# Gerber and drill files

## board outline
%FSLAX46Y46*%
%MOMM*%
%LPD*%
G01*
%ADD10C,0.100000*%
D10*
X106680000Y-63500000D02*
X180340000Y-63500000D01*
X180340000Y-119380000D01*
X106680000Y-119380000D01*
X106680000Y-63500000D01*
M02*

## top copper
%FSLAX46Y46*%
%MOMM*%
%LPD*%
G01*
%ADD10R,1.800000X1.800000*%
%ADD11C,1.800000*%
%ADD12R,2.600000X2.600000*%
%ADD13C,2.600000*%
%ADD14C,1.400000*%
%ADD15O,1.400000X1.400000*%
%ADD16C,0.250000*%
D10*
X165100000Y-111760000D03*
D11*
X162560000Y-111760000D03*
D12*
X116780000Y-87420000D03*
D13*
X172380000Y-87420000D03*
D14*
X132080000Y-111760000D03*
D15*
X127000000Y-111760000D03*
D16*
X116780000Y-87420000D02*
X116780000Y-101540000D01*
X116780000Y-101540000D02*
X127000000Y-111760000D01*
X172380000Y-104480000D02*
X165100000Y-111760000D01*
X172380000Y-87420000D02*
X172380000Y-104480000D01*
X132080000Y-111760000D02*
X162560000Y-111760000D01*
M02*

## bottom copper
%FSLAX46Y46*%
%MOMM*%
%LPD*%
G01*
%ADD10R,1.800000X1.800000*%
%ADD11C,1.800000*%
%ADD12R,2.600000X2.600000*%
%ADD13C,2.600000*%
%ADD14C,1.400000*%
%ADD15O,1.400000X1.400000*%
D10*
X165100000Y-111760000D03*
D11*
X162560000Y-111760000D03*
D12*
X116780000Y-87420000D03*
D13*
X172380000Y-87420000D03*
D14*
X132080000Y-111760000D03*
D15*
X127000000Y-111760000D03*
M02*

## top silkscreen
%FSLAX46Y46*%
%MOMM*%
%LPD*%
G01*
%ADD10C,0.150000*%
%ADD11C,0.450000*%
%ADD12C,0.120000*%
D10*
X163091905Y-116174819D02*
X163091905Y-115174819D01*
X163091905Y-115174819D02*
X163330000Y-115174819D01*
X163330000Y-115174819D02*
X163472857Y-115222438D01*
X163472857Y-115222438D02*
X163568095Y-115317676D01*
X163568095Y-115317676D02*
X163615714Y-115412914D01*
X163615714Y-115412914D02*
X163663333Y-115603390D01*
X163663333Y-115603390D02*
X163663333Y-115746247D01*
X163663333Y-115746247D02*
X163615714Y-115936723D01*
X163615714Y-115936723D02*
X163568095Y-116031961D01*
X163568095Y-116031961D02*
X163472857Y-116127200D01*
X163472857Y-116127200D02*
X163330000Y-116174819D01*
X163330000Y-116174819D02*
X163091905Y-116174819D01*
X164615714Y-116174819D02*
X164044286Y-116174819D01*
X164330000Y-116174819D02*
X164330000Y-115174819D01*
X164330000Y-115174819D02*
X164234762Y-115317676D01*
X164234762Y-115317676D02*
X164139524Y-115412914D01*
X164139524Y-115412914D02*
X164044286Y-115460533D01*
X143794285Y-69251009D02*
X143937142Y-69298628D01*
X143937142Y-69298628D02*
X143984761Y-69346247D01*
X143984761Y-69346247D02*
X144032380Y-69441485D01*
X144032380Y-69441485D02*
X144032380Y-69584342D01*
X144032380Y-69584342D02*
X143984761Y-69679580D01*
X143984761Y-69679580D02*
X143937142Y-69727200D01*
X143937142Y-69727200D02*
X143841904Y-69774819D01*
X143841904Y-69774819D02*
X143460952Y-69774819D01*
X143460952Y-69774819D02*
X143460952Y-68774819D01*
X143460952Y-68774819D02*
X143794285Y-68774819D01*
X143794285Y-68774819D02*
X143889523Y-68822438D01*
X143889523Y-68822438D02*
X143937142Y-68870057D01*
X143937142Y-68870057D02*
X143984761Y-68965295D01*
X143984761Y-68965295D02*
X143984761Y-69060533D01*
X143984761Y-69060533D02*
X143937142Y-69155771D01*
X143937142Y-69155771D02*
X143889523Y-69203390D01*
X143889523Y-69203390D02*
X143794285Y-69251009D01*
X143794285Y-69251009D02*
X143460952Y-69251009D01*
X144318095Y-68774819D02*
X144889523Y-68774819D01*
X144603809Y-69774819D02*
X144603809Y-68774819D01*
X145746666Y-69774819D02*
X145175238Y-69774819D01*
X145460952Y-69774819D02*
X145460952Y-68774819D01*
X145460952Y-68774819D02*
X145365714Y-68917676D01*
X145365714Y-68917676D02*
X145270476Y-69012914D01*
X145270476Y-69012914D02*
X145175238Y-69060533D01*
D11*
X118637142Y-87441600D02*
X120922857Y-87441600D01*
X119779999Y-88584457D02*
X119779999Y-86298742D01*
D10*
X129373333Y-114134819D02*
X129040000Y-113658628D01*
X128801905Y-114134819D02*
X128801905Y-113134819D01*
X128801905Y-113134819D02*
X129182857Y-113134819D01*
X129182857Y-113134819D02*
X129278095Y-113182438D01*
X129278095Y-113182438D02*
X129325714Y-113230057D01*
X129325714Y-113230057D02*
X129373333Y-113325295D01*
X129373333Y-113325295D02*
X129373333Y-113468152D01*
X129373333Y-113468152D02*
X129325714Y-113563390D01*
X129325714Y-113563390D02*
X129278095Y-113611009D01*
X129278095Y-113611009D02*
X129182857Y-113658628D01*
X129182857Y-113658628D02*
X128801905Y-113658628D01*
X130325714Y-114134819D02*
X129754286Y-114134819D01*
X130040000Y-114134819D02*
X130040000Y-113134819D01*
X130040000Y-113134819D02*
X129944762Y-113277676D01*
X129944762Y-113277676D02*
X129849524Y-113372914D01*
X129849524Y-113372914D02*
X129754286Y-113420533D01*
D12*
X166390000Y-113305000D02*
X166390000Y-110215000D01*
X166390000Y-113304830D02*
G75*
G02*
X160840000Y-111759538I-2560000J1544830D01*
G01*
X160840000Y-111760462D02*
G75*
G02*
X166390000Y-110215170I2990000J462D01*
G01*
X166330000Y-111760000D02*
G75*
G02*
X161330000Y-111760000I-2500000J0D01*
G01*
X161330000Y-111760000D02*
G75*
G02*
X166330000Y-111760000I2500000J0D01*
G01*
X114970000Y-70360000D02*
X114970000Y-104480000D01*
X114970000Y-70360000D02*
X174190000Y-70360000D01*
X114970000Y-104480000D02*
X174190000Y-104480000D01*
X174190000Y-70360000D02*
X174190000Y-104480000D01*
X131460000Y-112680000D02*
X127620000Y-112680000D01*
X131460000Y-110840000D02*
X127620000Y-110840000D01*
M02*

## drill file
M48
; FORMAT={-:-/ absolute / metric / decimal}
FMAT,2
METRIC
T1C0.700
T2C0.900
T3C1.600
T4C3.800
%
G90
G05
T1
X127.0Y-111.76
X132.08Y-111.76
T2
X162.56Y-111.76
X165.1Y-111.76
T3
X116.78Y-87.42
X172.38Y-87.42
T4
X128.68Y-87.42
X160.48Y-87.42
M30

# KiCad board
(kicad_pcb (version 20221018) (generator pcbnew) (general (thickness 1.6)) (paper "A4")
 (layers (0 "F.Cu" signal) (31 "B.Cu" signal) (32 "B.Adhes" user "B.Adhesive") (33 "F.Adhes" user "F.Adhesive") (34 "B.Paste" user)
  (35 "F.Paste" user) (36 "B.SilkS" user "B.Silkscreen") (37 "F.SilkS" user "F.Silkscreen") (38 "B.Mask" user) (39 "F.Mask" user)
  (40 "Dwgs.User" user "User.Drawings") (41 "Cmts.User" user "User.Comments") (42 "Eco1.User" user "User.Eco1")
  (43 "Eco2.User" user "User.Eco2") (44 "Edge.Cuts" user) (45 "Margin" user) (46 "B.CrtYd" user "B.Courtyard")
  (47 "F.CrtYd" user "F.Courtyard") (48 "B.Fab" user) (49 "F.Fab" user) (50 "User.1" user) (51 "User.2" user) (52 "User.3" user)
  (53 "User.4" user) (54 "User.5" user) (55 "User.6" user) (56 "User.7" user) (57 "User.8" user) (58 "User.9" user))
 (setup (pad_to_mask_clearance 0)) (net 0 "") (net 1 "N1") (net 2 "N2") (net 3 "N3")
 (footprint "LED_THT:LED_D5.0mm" (layer "F.Cu") (at 165.1 111.76 180)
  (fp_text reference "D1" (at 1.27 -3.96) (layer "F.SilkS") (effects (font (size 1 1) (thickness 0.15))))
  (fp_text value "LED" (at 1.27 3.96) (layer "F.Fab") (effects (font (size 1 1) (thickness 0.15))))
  (fp_line (start -1.29 -1.545) (end -1.29 1.545) (stroke (width 0.12) (type solid)) (layer "F.SilkS"))
  (fp_arc (start -1.29 -1.54483) (mid 2.072002 -2.880433) (end 4.26 0.000462) (stroke (width 0.12) (type solid)) (layer "F.SilkS"))
  (fp_arc (start 4.26 -0.000462) (mid 2.072002 2.880433) (end -1.29 1.54483) (stroke (width 0.12) (type solid)) (layer "F.SilkS"))
  (fp_circle (center 1.27 0) (end 3.77 0) (stroke (width 0.12) (type solid)) (fill none) (layer "F.SilkS"))
  (pad "1" thru_hole rect (at 0 0 180) (size 1.8 1.8) (drill 0.9) (layers "*.Cu" "*.Mask") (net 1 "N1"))
  (pad "2" thru_hole circle (at 2.54 0 180) (size 1.8 1.8) (drill 0.9) (layers "*.Cu" "*.Mask") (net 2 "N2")))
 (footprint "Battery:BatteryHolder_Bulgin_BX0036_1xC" (layer "F.Cu") (at 116.78 87.42)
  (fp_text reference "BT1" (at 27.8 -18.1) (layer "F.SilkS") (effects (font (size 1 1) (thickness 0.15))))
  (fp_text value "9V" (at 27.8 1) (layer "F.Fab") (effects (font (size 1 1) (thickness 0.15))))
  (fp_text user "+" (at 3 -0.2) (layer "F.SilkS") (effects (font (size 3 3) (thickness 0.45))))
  (fp_line (start -1.81 -17.06) (end -1.81 17.06) (stroke (width 0.12) (type solid)) (layer "F.SilkS"))
  (fp_line (start -1.81 -17.06) (end 57.41 -17.06) (stroke (width 0.12) (type solid)) (layer "F.SilkS"))
  (fp_line (start -1.81 17.06) (end 57.41 17.06) (stroke (width 0.12) (type solid)) (layer "F.SilkS"))
  (fp_line (start 57.41 -17.06) (end 57.41 17.06) (stroke (width 0.12) (type solid)) (layer "F.SilkS"))
  (pad "" np_thru_hole circle (at 11.9 0) (size 3.8 3.8) (drill 3.8) (layers "*.Cu" "*.Mask"))
  (pad "" np_thru_hole circle (at 43.7 0) (size 3.8 3.8) (drill 3.8) (layers "*.Cu" "*.Mask"))
  (pad "1" thru_hole rect (at 0 0) (size 2.6 2.6) (drill 1.6) (layers "*.Cu" "*.Mask") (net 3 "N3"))
  (pad "2" thru_hole circle (at 55.6 0) (size 2.6 2.6) (drill 1.6) (layers "*.Cu" "*.Mask") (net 1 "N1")))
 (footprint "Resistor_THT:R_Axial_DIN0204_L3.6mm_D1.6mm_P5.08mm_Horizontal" (layer "F.Cu") (at 132.08 111.76 180)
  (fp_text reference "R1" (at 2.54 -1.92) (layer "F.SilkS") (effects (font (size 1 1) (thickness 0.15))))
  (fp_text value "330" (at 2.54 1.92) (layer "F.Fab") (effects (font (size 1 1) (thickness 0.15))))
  (fp_line (start 0.62 -0.92) (end 4.46 -0.92) (stroke (width 0.12) (type solid)) (layer "F.SilkS"))
  (fp_line (start 0.62 0.92) (end 4.46 0.92) (stroke (width 0.12) (type solid)) (layer "F.SilkS"))
  (pad "1" thru_hole circle (at 0 0 180) (size 1.4 1.4) (drill 0.7) (layers "*.Cu" "*.Mask") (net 2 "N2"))
  (pad "2" thru_hole oval (at 5.08 0 180) (size 1.4 1.4) (drill 0.7) (layers "*.Cu" "*.Mask") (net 3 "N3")))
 (gr_rect (start 106.68 63.5) (end 180.34 119.38) (stroke (width 0.1) (type default)) (fill none) (layer "Edge.Cuts"))
 (segment (start 116.78 87.42) (end 116.78 101.54) (width 0.25) (layer "F.Cu") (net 3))
 (segment (start 116.78 101.54) (end 127 111.76) (width 0.25) (layer "F.Cu") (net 3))
 (segment (start 172.38 104.48) (end 165.1 111.76) (width 0.25) (layer "F.Cu") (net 1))
 (segment (start 172.38 87.42) (end 172.38 104.48) (width 0.25) (layer "F.Cu") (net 1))
 (segment (start 132.08 111.76) (end 162.56 111.76) (width 0.25) (layer "F.Cu") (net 2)))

